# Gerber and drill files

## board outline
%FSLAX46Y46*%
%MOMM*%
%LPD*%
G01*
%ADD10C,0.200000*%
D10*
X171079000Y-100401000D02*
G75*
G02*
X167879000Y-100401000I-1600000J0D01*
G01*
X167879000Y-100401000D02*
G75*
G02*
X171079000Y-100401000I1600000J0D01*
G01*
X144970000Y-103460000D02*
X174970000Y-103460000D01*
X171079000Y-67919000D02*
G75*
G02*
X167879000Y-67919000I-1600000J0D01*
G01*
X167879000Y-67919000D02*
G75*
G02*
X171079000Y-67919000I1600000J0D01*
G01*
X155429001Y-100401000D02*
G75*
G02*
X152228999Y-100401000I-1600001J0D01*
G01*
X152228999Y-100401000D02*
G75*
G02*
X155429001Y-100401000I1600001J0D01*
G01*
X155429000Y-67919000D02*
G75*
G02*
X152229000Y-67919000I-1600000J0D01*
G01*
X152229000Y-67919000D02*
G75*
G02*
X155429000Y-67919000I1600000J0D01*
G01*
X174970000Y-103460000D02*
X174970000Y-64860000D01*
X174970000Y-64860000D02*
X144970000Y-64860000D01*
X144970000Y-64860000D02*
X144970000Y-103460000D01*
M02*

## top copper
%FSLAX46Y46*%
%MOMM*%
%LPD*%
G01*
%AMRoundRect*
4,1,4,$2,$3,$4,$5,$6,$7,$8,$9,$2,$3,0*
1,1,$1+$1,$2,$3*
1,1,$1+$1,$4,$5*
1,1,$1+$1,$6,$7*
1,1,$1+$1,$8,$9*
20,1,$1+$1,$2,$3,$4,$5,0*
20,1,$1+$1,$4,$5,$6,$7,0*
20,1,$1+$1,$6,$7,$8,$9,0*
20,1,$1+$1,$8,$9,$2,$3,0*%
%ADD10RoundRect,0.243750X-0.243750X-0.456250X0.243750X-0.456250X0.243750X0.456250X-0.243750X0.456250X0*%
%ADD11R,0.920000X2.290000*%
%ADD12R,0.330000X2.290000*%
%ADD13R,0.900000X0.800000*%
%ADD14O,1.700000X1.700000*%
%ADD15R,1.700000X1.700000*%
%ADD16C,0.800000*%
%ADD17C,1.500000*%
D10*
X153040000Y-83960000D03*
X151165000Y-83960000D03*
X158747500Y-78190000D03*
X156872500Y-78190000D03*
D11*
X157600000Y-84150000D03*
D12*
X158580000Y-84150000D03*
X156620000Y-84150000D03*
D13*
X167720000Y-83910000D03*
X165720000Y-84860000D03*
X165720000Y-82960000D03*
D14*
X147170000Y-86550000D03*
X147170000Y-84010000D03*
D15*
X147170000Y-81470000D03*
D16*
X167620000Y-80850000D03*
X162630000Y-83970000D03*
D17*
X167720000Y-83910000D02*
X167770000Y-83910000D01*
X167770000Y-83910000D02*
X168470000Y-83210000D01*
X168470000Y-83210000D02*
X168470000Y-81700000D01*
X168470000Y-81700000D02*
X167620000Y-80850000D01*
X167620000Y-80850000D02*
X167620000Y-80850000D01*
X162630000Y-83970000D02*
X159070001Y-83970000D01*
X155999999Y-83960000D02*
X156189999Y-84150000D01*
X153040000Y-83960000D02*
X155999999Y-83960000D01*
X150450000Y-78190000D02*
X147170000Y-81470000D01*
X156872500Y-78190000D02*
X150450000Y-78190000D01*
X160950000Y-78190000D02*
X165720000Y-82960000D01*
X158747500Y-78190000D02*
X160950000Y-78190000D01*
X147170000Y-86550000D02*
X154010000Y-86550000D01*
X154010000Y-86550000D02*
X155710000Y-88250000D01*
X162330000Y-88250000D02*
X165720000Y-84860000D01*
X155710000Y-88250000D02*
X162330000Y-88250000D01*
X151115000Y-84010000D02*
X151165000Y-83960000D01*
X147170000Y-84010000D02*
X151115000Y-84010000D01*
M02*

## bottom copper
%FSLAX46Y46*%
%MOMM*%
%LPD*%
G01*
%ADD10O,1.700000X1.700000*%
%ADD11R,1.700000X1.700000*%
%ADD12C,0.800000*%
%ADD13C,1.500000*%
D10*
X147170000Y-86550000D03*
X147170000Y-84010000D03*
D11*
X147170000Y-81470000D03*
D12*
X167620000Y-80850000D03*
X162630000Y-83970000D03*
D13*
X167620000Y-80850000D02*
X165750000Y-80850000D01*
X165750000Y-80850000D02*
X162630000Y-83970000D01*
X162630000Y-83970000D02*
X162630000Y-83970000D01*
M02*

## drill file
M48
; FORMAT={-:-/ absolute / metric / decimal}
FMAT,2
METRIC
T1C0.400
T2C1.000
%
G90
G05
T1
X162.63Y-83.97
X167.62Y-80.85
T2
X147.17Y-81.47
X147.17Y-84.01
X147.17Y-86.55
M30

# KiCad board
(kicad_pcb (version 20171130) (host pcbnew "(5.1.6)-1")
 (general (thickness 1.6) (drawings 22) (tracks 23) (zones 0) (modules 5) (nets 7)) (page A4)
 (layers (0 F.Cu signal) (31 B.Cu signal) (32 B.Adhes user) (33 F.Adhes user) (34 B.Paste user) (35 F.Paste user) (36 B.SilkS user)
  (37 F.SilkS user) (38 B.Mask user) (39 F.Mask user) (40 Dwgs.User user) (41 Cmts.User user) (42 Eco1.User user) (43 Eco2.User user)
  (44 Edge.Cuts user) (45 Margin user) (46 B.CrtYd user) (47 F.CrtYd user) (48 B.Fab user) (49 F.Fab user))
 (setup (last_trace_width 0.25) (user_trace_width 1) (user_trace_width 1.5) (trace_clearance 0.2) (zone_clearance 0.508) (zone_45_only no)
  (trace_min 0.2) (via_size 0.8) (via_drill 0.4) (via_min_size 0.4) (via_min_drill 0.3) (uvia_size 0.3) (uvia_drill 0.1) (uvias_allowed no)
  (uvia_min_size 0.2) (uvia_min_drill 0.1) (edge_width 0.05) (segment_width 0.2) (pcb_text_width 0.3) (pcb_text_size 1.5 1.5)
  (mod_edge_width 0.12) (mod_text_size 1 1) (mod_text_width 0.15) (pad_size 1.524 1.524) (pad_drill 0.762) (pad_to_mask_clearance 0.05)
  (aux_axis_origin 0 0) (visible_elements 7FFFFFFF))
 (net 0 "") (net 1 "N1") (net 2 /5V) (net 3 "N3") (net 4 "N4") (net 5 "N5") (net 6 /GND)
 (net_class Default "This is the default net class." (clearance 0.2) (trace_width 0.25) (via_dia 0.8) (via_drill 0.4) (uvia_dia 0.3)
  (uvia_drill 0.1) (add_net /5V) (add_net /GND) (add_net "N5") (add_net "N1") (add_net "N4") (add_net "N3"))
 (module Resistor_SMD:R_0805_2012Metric (layer F.Cu) (at 152.1025 83.96)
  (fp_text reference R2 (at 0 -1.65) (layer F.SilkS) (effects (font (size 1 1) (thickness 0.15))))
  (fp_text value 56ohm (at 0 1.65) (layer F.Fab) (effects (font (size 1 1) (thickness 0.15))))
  (pad 2 smd roundrect (at 0.9375 0) (size 0.975 1.4) (layers F.Cu F.Paste F.Mask) (roundrect_rratio 0.25) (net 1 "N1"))
  (pad 1 smd roundrect (at -0.9375 0) (size 0.975 1.4) (layers F.Cu F.Paste F.Mask) (roundrect_rratio 0.25) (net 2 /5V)))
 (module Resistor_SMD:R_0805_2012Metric (layer F.Cu) (at 157.81 78.19)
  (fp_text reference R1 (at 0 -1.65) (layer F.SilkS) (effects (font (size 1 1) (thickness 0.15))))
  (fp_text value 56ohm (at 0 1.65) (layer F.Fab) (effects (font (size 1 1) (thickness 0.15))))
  (pad 2 smd roundrect (at 0.9375 0) (size 0.975 1.4) (layers F.Cu F.Paste F.Mask) (roundrect_rratio 0.25) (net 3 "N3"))
  (pad 1 smd roundrect (at -0.9375 0) (size 0.975 1.4) (layers F.Cu F.Paste F.Mask) (roundrect_rratio 0.25) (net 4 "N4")))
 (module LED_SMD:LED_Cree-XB (layer F.Cu) (at 157.6 84.15 180)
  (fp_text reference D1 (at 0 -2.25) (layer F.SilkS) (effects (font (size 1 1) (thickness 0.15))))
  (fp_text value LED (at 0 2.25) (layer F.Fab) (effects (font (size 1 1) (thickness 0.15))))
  (pad "" smd rect (at 0 0.55 180) (size 0.85 0.85) (layers F.Paste))
  (pad "" smd rect (at 0 -0.55 180) (size 0.85 0.85) (layers F.Paste))
  (pad 3 smd rect (at 0 0 180) (size 0.92 2.29) (layers F.Cu F.Mask))
  (pad 1 smd rect (at -0.98 0 180) (size 0.33 2.29) (layers F.Cu F.Paste F.Mask) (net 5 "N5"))
  (pad 2 smd rect (at 0.98 0 180) (size 0.33 2.29) (layers F.Cu F.Paste F.Mask) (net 1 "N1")))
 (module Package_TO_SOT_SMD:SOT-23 (layer F.Cu) (at 166.72 83.91)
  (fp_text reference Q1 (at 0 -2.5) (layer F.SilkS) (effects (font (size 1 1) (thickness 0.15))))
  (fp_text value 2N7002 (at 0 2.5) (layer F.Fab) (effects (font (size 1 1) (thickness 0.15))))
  (pad 3 smd rect (at 1 0) (size 0.9 0.8) (layers F.Cu F.Paste F.Mask) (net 5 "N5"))
  (pad 2 smd rect (at -1 0.95) (size 0.9 0.8) (layers F.Cu F.Paste F.Mask) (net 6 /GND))
  (pad 1 smd rect (at -1 -0.95) (size 0.9 0.8) (layers F.Cu F.Paste F.Mask) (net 3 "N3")))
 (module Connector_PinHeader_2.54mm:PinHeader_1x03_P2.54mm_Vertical (layer F.Cu) (at 147.17 81.47)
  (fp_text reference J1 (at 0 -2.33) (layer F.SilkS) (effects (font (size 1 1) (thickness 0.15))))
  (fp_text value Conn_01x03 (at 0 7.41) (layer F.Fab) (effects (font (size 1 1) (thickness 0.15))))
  (pad 3 thru_hole oval (at 0 5.08) (size 1.7 1.7) (drill 1) (layers *.Cu *.Mask) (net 6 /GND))
  (pad 2 thru_hole oval (at 0 2.54) (size 1.7 1.7) (drill 1) (layers *.Cu *.Mask) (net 2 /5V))
  (pad 1 thru_hole rect (at 0 0) (size 1.7 1.7) (drill 1) (layers *.Cu *.Mask) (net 4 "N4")))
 (gr_circle (center 169.479 100.401) (end 171.079 100.401) (layer Edge.Cuts) (width 0.2))
 (gr_line (start 144.97 103.46) (end 174.97 103.46) (layer Edge.Cuts) (width 0.2))
 (gr_circle (center 169.479 67.919) (end 171.079 67.919) (layer Edge.Cuts) (width 0.2))
 (gr_circle (center 153.829 100.401) (end 155.429001 100.401) (layer Edge.Cuts) (width 0.2))
 (gr_circle (center 153.829 67.919) (end 155.429 67.919) (layer Edge.Cuts) (width 0.2))
 (gr_line (start 174.97 103.46) (end 174.97 64.86) (layer Edge.Cuts) (width 0.2))
 (gr_line (start 174.97 64.86) (end 144.97 64.86) (layer Edge.Cuts) (width 0.2))
 (gr_line (start 144.97 64.86) (end 144.97 103.46) (layer Edge.Cuts) (width 0.2))
 (segment (start 167.72 83.91) (end 167.77 83.91) (width 1.5) (layer F.Cu) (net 5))
 (segment (start 167.77 83.91) (end 168.47 83.21) (width 1.5) (layer F.Cu) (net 5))
 (segment (start 168.47 83.21) (end 168.47 81.7) (width 1.5) (layer F.Cu) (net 5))
 (segment (start 168.47 81.7) (end 167.62 80.85) (width 1.5) (layer F.Cu) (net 5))
 (segment (start 167.62 80.85) (end 167.62 80.85) (width 1.5) (layer F.Cu) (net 5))
 (via (at 167.62 80.85) (size 0.8) (drill 0.4) (layers F.Cu B.Cu) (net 5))
 (segment (start 167.62 80.85) (end 165.75 80.85) (width 1.5) (layer B.Cu) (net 5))
 (segment (start 165.75 80.85) (end 162.63 83.97) (width 1.5) (layer B.Cu) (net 5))
 (segment (start 162.63 83.97) (end 162.63 83.97) (width 1.5) (layer B.Cu) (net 5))
 (via (at 162.63 83.97) (size 0.8) (drill 0.4) (layers F.Cu B.Cu) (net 5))
 (segment (start 162.63 83.97) (end 159.070001 83.97) (width 1.5) (layer F.Cu) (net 5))
 (segment (start 155.999999 83.96) (end 156.189999 84.15) (width 1.5) (layer F.Cu) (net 1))
 (segment (start 153.04 83.96) (end 155.999999 83.96) (width 1.5) (layer F.Cu) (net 1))
 (segment (start 150.45 78.19) (end 147.17 81.47) (width 1.5) (layer F.Cu) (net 4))
 (segment (start 156.8725 78.19) (end 150.45 78.19) (width 1.5) (layer F.Cu) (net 4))
 (segment (start 160.95 78.19) (end 165.72 82.96) (width 1.5) (layer F.Cu) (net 3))
 (segment (start 158.7475 78.19) (end 160.95 78.19) (width 1.5) (layer F.Cu) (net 3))
 (segment (start 147.17 86.55) (end 154.01 86.55) (width 1.5) (layer F.Cu) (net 6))
 (segment (start 154.01 86.55) (end 155.71 88.25) (width 1.5) (layer F.Cu) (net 6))
 (segment (start 162.33 88.25) (end 165.72 84.86) (width 1.5) (layer F.Cu) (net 6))
 (segment (start 155.71 88.25) (end 162.33 88.25) (width 1.5) (layer F.Cu) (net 6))
 (segment (start 151.115 84.01) (end 151.165 83.96) (width 1.5) (layer F.Cu) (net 2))
 (segment (start 147.17 84.01) (end 151.115 84.01) (width 1.5) (layer F.Cu) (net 2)))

